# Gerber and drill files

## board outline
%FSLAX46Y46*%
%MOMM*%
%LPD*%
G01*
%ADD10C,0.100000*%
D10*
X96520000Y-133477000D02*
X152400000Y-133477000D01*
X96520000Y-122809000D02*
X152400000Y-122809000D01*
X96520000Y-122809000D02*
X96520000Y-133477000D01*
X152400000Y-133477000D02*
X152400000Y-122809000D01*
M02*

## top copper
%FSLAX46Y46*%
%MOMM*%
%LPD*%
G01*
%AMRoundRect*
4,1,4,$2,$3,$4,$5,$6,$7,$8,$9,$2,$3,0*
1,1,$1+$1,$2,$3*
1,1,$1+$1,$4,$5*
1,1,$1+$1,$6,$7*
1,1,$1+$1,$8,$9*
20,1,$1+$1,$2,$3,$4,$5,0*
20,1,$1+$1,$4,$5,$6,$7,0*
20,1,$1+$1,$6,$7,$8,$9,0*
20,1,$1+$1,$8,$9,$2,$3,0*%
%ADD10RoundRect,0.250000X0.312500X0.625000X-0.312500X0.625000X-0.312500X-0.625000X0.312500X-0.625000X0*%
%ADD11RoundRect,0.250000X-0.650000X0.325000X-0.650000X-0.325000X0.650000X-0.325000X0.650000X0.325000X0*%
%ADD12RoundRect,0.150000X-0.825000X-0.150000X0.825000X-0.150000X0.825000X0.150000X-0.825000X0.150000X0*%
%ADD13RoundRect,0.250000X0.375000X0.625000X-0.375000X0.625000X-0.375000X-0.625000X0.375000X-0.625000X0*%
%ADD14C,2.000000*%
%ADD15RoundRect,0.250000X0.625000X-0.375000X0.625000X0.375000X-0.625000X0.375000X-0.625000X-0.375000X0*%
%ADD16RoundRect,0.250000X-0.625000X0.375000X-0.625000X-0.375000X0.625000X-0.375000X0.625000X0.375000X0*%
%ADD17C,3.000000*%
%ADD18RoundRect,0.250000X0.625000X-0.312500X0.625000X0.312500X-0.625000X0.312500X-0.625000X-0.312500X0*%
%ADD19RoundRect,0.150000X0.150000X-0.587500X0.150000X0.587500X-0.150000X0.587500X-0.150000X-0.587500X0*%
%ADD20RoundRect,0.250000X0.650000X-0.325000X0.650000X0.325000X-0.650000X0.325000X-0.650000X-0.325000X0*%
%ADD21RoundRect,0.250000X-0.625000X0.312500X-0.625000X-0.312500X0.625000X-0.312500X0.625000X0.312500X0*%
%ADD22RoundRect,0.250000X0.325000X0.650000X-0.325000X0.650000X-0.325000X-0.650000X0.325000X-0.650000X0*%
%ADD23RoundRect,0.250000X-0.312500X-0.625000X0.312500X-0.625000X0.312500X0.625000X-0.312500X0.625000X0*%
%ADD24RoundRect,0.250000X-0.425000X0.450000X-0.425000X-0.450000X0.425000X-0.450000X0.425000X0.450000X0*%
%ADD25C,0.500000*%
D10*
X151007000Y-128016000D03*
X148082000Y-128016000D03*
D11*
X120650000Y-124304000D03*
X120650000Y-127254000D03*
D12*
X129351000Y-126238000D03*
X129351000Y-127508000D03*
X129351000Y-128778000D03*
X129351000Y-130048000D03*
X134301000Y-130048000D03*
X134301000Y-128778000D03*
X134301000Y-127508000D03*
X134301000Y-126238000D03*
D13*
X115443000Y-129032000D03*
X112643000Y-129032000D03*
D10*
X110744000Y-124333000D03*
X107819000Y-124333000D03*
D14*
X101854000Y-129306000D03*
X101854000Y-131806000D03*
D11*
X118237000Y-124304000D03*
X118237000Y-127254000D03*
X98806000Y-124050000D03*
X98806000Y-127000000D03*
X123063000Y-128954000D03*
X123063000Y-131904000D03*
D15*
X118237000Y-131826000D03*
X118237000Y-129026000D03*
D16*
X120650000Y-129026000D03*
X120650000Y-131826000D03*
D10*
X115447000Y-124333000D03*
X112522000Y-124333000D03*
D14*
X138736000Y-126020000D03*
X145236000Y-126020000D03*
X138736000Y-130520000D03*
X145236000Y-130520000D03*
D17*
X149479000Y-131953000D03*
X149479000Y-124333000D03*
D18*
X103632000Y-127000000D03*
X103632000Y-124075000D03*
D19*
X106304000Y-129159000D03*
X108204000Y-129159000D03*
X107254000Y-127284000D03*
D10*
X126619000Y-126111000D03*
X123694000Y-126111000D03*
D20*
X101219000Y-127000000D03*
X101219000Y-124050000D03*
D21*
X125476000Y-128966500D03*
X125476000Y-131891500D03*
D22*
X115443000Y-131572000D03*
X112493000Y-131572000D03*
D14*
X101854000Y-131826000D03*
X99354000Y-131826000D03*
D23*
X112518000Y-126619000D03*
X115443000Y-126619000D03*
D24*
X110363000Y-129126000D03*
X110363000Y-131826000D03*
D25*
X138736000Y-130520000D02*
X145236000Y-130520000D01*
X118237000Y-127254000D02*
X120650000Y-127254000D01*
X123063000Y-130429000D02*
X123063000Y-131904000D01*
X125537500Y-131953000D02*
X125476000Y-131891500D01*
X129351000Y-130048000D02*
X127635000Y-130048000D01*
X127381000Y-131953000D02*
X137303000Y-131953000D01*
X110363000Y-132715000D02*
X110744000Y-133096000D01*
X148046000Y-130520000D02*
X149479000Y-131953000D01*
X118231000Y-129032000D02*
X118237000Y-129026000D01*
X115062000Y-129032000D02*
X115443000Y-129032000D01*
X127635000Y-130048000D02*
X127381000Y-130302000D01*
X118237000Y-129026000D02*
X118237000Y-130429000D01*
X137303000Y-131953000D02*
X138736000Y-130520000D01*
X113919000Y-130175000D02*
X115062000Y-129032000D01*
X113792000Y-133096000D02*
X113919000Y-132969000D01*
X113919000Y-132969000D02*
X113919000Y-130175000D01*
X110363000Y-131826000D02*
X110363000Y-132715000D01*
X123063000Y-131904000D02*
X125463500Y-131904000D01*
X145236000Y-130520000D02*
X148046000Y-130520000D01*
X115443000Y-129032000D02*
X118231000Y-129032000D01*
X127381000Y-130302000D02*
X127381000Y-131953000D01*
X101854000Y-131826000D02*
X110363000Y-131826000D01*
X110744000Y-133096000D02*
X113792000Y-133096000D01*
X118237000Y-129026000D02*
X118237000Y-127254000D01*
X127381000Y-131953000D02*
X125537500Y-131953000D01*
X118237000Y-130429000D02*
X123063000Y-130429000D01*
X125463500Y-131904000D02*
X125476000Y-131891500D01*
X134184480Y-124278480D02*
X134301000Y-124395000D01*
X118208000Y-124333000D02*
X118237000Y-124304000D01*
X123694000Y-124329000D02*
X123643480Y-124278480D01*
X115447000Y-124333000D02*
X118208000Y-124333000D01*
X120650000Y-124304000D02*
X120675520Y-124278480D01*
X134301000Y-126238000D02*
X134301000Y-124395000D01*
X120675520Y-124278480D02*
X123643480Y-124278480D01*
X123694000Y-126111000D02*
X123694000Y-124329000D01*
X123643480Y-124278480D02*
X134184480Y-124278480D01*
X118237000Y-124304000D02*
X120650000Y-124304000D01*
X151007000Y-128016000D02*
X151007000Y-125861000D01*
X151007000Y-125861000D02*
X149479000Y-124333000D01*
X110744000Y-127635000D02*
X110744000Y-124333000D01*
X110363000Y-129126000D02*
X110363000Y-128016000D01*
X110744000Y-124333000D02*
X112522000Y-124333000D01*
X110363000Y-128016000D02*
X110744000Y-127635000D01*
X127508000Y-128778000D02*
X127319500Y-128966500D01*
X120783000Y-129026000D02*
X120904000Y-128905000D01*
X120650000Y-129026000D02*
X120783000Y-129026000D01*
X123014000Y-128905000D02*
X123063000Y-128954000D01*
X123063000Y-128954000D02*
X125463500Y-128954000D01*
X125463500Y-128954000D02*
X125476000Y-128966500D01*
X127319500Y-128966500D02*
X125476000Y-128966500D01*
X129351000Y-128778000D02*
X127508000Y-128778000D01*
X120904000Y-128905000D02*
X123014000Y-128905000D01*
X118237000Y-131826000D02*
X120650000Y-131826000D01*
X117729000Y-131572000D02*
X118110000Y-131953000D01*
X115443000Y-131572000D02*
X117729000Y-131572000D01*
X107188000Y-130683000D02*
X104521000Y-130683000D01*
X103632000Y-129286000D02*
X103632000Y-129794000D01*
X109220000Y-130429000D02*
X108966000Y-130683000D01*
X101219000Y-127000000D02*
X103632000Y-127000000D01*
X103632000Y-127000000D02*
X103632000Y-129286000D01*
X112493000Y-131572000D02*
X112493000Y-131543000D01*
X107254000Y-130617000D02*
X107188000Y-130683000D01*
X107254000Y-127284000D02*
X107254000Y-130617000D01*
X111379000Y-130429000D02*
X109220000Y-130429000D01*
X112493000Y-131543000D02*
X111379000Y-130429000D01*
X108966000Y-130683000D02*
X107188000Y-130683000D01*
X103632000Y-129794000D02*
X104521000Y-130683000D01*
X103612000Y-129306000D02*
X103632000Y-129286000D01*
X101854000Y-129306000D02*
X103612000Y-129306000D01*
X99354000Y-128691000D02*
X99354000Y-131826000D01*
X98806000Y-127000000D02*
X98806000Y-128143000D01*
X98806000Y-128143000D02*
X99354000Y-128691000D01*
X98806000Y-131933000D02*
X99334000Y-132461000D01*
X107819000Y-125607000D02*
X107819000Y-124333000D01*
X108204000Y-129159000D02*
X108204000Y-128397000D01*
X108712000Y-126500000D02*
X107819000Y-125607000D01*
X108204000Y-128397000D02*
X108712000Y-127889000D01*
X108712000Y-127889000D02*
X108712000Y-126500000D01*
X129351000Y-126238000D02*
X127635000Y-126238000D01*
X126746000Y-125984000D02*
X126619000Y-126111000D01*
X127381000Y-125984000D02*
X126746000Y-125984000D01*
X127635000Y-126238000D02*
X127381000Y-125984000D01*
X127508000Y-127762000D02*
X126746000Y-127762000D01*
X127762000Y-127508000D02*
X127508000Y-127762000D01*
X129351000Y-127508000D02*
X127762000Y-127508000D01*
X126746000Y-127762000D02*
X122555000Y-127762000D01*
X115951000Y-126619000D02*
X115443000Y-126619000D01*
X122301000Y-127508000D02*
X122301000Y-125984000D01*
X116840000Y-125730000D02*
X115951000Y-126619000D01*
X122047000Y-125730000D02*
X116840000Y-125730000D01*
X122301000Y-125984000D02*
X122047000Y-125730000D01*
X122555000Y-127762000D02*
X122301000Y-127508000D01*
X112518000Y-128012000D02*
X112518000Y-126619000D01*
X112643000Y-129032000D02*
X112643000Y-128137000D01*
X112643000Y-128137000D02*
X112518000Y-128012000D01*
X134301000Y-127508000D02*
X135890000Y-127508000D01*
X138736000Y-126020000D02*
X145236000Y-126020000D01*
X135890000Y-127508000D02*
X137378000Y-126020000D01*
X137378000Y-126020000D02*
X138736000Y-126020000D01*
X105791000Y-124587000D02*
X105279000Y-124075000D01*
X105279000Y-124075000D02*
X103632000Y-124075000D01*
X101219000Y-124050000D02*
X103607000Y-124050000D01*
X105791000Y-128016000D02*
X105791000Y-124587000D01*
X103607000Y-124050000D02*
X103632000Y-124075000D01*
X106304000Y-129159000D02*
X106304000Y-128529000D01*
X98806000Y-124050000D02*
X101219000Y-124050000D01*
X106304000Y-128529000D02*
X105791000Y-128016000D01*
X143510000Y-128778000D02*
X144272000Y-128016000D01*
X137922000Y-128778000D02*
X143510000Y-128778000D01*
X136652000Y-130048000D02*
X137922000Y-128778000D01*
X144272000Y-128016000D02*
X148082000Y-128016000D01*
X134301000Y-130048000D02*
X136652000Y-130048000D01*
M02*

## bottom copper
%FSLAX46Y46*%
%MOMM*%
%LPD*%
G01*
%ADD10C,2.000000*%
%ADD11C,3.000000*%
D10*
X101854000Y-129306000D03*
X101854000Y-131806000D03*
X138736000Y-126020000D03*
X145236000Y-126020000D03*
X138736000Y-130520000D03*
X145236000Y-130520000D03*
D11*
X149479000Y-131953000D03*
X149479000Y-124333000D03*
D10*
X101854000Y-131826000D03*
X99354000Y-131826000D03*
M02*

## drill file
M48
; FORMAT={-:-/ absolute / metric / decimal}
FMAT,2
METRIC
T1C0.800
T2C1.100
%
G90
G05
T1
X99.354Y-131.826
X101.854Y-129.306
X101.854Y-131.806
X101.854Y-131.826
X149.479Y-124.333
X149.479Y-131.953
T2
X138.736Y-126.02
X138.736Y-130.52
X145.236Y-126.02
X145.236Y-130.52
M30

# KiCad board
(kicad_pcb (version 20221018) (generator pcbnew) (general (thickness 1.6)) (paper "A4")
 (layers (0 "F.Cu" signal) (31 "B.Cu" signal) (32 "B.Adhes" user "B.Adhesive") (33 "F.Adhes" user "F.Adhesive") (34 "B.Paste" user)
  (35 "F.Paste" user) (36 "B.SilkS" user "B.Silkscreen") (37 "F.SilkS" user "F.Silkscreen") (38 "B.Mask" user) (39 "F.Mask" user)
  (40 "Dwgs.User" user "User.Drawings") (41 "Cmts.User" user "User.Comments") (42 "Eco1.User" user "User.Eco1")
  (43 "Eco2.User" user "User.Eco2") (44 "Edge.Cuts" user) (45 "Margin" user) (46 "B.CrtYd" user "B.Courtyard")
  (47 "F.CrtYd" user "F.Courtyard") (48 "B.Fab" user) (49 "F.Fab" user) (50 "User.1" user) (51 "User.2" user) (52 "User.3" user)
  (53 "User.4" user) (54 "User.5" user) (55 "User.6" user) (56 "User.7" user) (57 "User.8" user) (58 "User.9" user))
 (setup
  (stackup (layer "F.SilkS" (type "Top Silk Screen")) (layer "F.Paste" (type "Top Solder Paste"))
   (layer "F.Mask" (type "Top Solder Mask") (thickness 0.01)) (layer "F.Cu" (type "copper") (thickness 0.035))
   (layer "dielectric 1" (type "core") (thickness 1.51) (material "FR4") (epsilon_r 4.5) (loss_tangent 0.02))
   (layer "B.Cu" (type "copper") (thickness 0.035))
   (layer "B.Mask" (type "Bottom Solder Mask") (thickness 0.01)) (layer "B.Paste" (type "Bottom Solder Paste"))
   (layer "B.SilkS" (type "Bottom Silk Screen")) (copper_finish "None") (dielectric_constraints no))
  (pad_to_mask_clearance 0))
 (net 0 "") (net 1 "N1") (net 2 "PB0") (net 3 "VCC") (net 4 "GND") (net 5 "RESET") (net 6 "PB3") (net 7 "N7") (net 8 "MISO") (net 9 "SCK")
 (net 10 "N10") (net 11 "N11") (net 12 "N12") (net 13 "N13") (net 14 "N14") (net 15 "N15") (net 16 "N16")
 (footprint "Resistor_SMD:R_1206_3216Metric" (layer "F.Cu") (at 149.5445 128.016 180)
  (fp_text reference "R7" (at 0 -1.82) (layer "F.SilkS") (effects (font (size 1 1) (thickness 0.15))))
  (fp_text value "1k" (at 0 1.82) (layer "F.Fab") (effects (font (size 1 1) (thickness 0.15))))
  (pad "1" smd roundrect (at -1.4625 0 180) (size 1.125 1.75) (layers "F.Cu" "F.Paste" "F.Mask") (roundrect_rratio 0.222222) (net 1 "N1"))
  (pad "2" smd roundrect (at 1.4625 0 180) (size 1.125 1.75) (layers "F.Cu" "F.Paste" "F.Mask") (roundrect_rratio 0.222222) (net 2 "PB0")))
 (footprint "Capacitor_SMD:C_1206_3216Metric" (layer "F.Cu") (at 120.65 125.779 -90)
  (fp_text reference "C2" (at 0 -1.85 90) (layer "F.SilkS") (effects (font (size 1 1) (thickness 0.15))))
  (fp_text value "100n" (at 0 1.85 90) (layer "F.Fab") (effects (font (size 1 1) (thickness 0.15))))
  (pad "1" smd roundrect (at -1.475 0 270) (size 1.15 1.8) (layers "F.Cu" "F.Paste" "F.Mask") (roundrect_rratio 0.2173913043) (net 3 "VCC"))
  (pad "2" smd roundrect (at 1.475 0 270) (size 1.15 1.8) (layers "F.Cu" "F.Paste" "F.Mask") (roundrect_rratio 0.2173913043) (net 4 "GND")))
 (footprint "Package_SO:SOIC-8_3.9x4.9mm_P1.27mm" (layer "F.Cu") (at 131.826 128.143)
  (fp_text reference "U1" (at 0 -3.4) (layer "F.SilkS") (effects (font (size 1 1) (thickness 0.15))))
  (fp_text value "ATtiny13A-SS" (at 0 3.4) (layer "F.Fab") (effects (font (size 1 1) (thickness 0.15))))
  (pad "1" smd roundrect (at -2.475 -1.905) (size 1.95 0.6) (layers "F.Cu" "F.Paste" "F.Mask") (roundrect_rratio 0.25) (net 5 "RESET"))
  (pad "2" smd roundrect (at -2.475 -0.635) (size 1.95 0.6) (layers "F.Cu" "F.Paste" "F.Mask") (roundrect_rratio 0.25) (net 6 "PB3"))
  (pad "3" smd roundrect (at -2.475 0.635) (size 1.95 0.6) (layers "F.Cu" "F.Paste" "F.Mask") (roundrect_rratio 0.25) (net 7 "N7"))
  (pad "4" smd roundrect (at -2.475 1.905) (size 1.95 0.6) (layers "F.Cu" "F.Paste" "F.Mask") (roundrect_rratio 0.25) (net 4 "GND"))
  (pad "5" smd roundrect (at 2.475 1.905) (size 1.95 0.6) (layers "F.Cu" "F.Paste" "F.Mask") (roundrect_rratio 0.25) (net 2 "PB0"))
  (pad "6" smd roundrect (at 2.475 0.635) (size 1.95 0.6) (layers "F.Cu" "F.Paste" "F.Mask") (roundrect_rratio 0.25) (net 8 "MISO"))
  (pad "7" smd roundrect (at 2.475 -0.635) (size 1.95 0.6) (layers "F.Cu" "F.Paste" "F.Mask") (roundrect_rratio 0.25) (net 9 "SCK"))
  (pad "8" smd roundrect (at 2.475 -1.905) (size 1.95 0.6) (layers "F.Cu" "F.Paste" "F.Mask") (roundrect_rratio 0.25) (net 3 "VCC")))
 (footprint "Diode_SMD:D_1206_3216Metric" (layer "F.Cu") (at 114.043 129.032 180)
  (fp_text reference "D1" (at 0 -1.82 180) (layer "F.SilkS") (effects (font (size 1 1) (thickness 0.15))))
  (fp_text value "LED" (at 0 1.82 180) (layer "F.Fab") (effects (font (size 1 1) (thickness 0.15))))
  (pad "1" smd roundrect (at -1.4 0 180) (size 1.25 1.75) (layers "F.Cu" "F.Paste" "F.Mask") (roundrect_rratio 0.2) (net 4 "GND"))
  (pad "2" smd roundrect (at 1.4 0 180) (size 1.25 1.75) (layers "F.Cu" "F.Paste" "F.Mask") (roundrect_rratio 0.2) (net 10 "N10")))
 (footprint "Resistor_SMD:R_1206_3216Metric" (layer "F.Cu") (at 109.2815 124.333 180)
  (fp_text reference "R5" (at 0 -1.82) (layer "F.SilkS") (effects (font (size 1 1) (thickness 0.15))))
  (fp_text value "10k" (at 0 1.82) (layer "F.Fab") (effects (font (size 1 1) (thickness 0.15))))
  (pad "1" smd roundrect (at -1.4625 0 180) (size 1.125 1.75) (layers "F.Cu" "F.Paste" "F.Mask") (roundrect_rratio 0.2222222222)
   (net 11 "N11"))
  (pad "2" smd roundrect (at 1.4625 0 180) (size 1.125 1.75) (layers "F.Cu" "F.Paste" "F.Mask") (roundrect_rratio 0.2222222222)
   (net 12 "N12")))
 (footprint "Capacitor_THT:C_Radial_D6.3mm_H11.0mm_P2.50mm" (layer "F.Cu") (at 101.854 129.306 -90)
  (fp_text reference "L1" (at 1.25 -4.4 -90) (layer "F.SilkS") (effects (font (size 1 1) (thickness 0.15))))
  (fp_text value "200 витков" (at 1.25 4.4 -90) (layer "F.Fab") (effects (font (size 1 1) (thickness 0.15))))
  (pad "1" thru_hole circle (at 0 0 270) (size 2 2) (drill 0.8) (layers "*.Cu" "*.Mask") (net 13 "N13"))
  (pad "2" thru_hole circle (at 2.5 0 270) (size 2 2) (drill 0.8) (layers "*.Cu" "*.Mask") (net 4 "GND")))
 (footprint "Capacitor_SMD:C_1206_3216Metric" (layer "F.Cu") (at 118.237 125.779 -90)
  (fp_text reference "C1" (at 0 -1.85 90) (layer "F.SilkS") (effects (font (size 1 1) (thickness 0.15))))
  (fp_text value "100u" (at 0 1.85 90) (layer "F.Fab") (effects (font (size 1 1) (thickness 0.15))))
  (pad "1" smd roundrect (at -1.475 0 270) (size 1.15 1.8) (layers "F.Cu" "F.Paste" "F.Mask") (roundrect_rratio 0.2173913043) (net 3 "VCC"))
  (pad "2" smd roundrect (at 1.475 0 270) (size 1.15 1.8) (layers "F.Cu" "F.Paste" "F.Mask") (roundrect_rratio 0.2173913043) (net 4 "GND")))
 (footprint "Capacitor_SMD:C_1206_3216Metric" (layer "F.Cu") (at 98.806 125.525 -90)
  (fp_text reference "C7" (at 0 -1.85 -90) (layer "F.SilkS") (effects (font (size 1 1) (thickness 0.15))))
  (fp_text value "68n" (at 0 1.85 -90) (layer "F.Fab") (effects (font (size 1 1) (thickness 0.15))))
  (pad "1" smd roundrect (at -1.475 0 270) (size 1.15 1.8) (layers "F.Cu" "F.Paste" "F.Mask") (roundrect_rratio 0.2173913043) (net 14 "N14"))
  (pad "2" smd roundrect (at 1.475 0 270) (size 1.15 1.8) (layers "F.Cu" "F.Paste" "F.Mask") (roundrect_rratio 0.2173913043) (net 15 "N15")))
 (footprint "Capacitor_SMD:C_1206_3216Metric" (layer "F.Cu") (at 123.063 130.429 -90)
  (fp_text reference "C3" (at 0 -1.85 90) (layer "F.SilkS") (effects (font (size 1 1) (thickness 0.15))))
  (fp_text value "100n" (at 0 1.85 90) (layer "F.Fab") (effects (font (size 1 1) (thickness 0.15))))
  (pad "1" smd roundrect (at -1.475 0 270) (size 1.15 1.8) (layers "F.Cu" "F.Paste" "F.Mask") (roundrect_rratio 0.2173913043) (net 7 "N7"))
  (pad "2" smd roundrect (at 1.475 0 270) (size 1.15 1.8) (layers "F.Cu" "F.Paste" "F.Mask") (roundrect_rratio 0.2173913043) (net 4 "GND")))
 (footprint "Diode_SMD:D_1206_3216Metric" (layer "F.Cu") (at 118.237 130.426 90)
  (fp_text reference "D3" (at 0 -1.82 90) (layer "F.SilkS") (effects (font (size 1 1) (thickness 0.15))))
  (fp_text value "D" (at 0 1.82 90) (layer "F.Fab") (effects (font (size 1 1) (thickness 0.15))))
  (pad "1" smd roundrect (at -1.4 0 90) (size 1.25 1.75) (layers "F.Cu" "F.Paste" "F.Mask") (roundrect_rratio 0.2) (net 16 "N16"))
  (pad "2" smd roundrect (at 1.4 0 90) (size 1.25 1.75) (layers "F.Cu" "F.Paste" "F.Mask") (roundrect_rratio 0.2) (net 4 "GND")))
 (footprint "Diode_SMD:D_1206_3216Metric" (layer "F.Cu") (at 120.65 130.426 -90)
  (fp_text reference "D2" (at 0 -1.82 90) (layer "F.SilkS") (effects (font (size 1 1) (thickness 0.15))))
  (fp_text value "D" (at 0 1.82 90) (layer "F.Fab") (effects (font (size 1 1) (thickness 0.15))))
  (pad "1" smd roundrect (at -1.4 0 270) (size 1.25 1.75) (layers "F.Cu" "F.Paste" "F.Mask") (roundrect_rratio 0.2) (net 7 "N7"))
  (pad "2" smd roundrect (at 1.4 0 270) (size 1.25 1.75) (layers "F.Cu" "F.Paste" "F.Mask") (roundrect_rratio 0.2) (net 16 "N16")))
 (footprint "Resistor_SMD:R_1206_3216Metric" (layer "F.Cu") (at 113.9845 124.333 180)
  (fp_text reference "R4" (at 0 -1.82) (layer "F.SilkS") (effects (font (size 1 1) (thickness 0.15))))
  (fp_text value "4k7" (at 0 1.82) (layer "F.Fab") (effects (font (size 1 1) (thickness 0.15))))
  (pad "1" smd roundrect (at -1.4625 0 180) (size 1.125 1.75) (layers "F.Cu" "F.Paste" "F.Mask") (roundrect_rratio 0.2222222222)
   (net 3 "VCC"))
  (pad "2" smd roundrect (at 1.4625 0 180) (size 1.125 1.75) (layers "F.Cu" "F.Paste" "F.Mask") (roundrect_rratio 0.2222222222)
   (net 11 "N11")))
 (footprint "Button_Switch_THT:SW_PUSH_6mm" (layer "F.Cu") (at 138.736 126.02)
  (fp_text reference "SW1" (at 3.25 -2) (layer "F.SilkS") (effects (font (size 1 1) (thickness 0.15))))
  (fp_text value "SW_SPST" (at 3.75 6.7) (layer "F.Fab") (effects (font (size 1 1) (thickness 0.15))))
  (pad "1" thru_hole circle (at 0 0 90) (size 2 2) (drill 1.1) (layers "*.Cu" "*.Mask") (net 9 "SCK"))
  (pad "1" thru_hole circle (at 6.5 0 90) (size 2 2) (drill 1.1) (layers "*.Cu" "*.Mask") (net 9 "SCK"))
  (pad "2" thru_hole circle (at 0 4.5 90) (size 2 2) (drill 1.1) (layers "*.Cu" "*.Mask") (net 4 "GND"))
  (pad "2" thru_hole circle (at 6.5 4.5 90) (size 2 2) (drill 1.1) (layers "*.Cu" "*.Mask") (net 4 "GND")))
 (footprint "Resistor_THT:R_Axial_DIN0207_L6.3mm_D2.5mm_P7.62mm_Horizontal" (layer "F.Cu") (at 149.479 131.953 90)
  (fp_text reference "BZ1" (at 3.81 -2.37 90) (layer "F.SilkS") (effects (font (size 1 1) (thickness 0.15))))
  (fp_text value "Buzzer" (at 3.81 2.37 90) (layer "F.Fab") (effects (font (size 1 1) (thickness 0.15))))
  (pad "1" thru_hole circle (at 0 0 90) (size 3 3) (drill 0.8) (layers "*.Cu" "*.Mask") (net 4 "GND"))
  (pad "2" thru_hole circle (at 7.62 0 90) (size 3 3) (drill 0.8) (layers "*.Cu" "*.Mask") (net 1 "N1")))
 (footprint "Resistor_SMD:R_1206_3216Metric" (layer "F.Cu") (at 103.632 125.5375 90)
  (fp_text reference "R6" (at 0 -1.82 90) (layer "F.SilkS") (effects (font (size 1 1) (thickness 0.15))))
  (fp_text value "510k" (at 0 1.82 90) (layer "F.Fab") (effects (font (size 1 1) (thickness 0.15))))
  (pad "1" smd roundrect (at -1.4625 0 90) (size 1.125 1.75) (layers "F.Cu" "F.Paste" "F.Mask") (roundrect_rratio 0.2222222222)
   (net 13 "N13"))
  (pad "2" smd roundrect (at 1.4625 0 90) (size 1.125 1.75) (layers "F.Cu" "F.Paste" "F.Mask") (roundrect_rratio 0.2222222222)
   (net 14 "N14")))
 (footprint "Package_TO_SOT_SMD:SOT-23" (layer "F.Cu") (at 107.254 128.2215 90)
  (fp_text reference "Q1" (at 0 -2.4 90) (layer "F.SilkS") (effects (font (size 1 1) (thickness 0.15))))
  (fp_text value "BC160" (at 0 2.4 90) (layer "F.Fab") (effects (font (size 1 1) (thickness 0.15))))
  (pad "1" smd roundrect (at -0.9375 -0.95 90) (size 1.475 0.6) (layers "F.Cu" "F.Paste" "F.Mask") (roundrect_rratio 0.25) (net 14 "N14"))
  (pad "2" smd roundrect (at -0.9375 0.95 90) (size 1.475 0.6) (layers "F.Cu" "F.Paste" "F.Mask") (roundrect_rratio 0.25) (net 12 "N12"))
  (pad "3" smd roundrect (at 0.9375 0 90) (size 1.475 0.6) (layers "F.Cu" "F.Paste" "F.Mask") (roundrect_rratio 0.25) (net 13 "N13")))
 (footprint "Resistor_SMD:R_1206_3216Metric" (layer "F.Cu") (at 125.1565 126.111 180)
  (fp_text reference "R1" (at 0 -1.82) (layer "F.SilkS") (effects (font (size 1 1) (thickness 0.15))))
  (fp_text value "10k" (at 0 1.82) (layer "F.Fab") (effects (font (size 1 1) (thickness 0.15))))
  (pad "1" smd roundrect (at -1.4625 0 180) (size 1.125 1.75) (layers "F.Cu" "F.Paste" "F.Mask") (roundrect_rratio 0.2222222222)
   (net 5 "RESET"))
  (pad "2" smd roundrect (at 1.4625 0 180) (size 1.125 1.75) (layers "F.Cu" "F.Paste" "F.Mask") (roundrect_rratio 0.2222222222)
   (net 3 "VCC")))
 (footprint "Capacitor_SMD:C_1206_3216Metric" (layer "F.Cu") (at 101.219 125.525 90)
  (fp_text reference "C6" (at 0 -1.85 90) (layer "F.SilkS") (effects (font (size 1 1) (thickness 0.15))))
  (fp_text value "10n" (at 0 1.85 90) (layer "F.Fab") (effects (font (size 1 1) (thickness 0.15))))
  (pad "1" smd roundrect (at -1.475 0 90) (size 1.15 1.8) (layers "F.Cu" "F.Paste" "F.Mask") (roundrect_rratio 0.2173913043) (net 13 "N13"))
  (pad "2" smd roundrect (at 1.475 0 90) (size 1.15 1.8) (layers "F.Cu" "F.Paste" "F.Mask") (roundrect_rratio 0.2173913043) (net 14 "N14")))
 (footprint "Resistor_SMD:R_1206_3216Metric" (layer "F.Cu") (at 125.476 130.429 -90)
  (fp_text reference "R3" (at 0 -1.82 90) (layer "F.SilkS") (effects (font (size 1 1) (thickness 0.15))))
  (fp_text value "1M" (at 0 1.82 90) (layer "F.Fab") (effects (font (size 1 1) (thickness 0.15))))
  (pad "1" smd roundrect (at -1.4625 0 270) (size 1.125 1.75) (layers "F.Cu" "F.Paste" "F.Mask") (roundrect_rratio 0.2222222222)
   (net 7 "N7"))
  (pad "2" smd roundrect (at 1.4625 0 270) (size 1.125 1.75) (layers "F.Cu" "F.Paste" "F.Mask") (roundrect_rratio 0.2222222222)
   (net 4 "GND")))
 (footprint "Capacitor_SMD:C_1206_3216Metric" (layer "F.Cu") (at 113.968 131.572 180)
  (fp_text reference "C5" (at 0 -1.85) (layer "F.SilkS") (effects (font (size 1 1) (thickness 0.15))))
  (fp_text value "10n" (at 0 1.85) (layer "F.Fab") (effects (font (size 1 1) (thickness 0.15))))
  (pad "1" smd roundrect (at -1.475 0 180) (size 1.15 1.8) (layers "F.Cu" "F.Paste" "F.Mask") (roundrect_rratio 0.2173913043) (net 16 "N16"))
  (pad "2" smd roundrect (at 1.475 0 180) (size 1.15 1.8) (layers "F.Cu" "F.Paste" "F.Mask") (roundrect_rratio 0.2173913043) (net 13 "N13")))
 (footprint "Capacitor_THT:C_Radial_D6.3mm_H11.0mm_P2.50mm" (layer "F.Cu") (at 101.854 131.826 180)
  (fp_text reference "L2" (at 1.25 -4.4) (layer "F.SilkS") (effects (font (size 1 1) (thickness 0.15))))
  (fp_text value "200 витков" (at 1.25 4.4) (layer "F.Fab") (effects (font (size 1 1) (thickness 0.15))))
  (pad "1" thru_hole circle (at 0 0 180) (size 2 2) (drill 0.8) (layers "*.Cu" "*.Mask") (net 4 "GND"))
  (pad "2" thru_hole circle (at 2.5 0 180) (size 2 2) (drill 0.8) (layers "*.Cu" "*.Mask") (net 15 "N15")))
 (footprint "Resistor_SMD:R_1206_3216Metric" (layer "F.Cu") (at 113.9805 126.619)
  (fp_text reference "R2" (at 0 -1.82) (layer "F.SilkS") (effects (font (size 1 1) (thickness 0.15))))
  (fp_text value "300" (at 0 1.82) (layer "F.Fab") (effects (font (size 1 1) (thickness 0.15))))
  (pad "1" smd roundrect (at -1.4625 0) (size 1.125 1.75) (layers "F.Cu" "F.Paste" "F.Mask") (roundrect_rratio 0.2222222222) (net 10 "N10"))
  (pad "2" smd roundrect (at 1.4625 0) (size 1.125 1.75) (layers "F.Cu" "F.Paste" "F.Mask") (roundrect_rratio 0.2222222222) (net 6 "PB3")))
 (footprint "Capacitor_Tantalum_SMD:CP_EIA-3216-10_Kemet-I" (layer "F.Cu") (at 110.363 130.476 -90)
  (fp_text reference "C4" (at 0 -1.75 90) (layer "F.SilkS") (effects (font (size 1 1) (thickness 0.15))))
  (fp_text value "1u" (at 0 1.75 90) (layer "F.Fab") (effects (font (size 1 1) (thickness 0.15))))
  (pad "1" smd roundrect (at -1.35 0 270) (size 1.4 1.35) (layers "F.Cu" "F.Paste" "F.Mask") (roundrect_rratio 0.1851851852) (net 11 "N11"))
  (pad "2" smd roundrect (at 1.35 0 270) (size 1.4 1.35) (layers "F.Cu" "F.Paste" "F.Mask") (roundrect_rratio 0.1851851852) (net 4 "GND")))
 (gr_line (start 96.52 133.477) (end 152.4 133.477) (stroke (width 0.1) (type solid)) (layer "Edge.Cuts"))
 (gr_line (start 96.52 122.809) (end 152.4 122.809) (stroke (width 0.1) (type solid)) (layer "Edge.Cuts"))
 (gr_line (start 96.52 122.809) (end 96.52 133.477) (stroke (width 0.1) (type solid)) (layer "Edge.Cuts"))
 (gr_line (start 152.4 133.477) (end 152.4 122.809) (stroke (width 0.1) (type solid)) (layer "Edge.Cuts"))
 (segment (start 138.736 130.52) (end 145.236 130.52) (width 0.5) (layer "F.Cu") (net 4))
 (segment (start 118.237 127.254) (end 120.65 127.254) (width 0.5) (layer "F.Cu") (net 4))
 (segment (start 123.063 130.429) (end 123.063 131.904) (width 0.5) (layer "F.Cu") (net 4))
 (segment (start 125.5375 131.953) (end 125.476 131.8915) (width 0.5) (layer "F.Cu") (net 4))
 (segment (start 129.351 130.048) (end 127.635 130.048) (width 0.5) (layer "F.Cu") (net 4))
 (segment (start 127.381 131.953) (end 137.303 131.953) (width 0.5) (layer "F.Cu") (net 4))
 (segment (start 110.363 132.715) (end 110.744 133.096) (width 0.5) (layer "F.Cu") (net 4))
 (segment (start 148.046 130.52) (end 149.479 131.953) (width 0.5) (layer "F.Cu") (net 4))
 (segment (start 118.231 129.032) (end 118.237 129.026) (width 0.5) (layer "F.Cu") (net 4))
 (segment (start 115.062 129.032) (end 115.443 129.032) (width 0.5) (layer "F.Cu") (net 4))
 (segment (start 127.635 130.048) (end 127.381 130.302) (width 0.5) (layer "F.Cu") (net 4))
 (segment (start 118.237 129.026) (end 118.237 130.429) (width 0.5) (layer "F.Cu") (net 4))
 (segment (start 137.303 131.953) (end 138.736 130.52) (width 0.5) (layer "F.Cu") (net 4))
 (segment (start 113.919 130.175) (end 115.062 129.032) (width 0.5) (layer "F.Cu") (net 4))
 (segment (start 113.792 133.096) (end 113.919 132.969) (width 0.5) (layer "F.Cu") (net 4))
 (segment (start 113.919 132.969) (end 113.919 130.175) (width 0.5) (layer "F.Cu") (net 4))
 (segment (start 110.363 131.826) (end 110.363 132.715) (width 0.5) (layer "F.Cu") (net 4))
 (segment (start 123.063 131.904) (end 125.4635 131.904) (width 0.5) (layer "F.Cu") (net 4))
 (segment (start 145.236 130.52) (end 148.046 130.52) (width 0.5) (layer "F.Cu") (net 4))
 (segment (start 115.443 129.032) (end 118.231 129.032) (width 0.5) (layer "F.Cu") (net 4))
 (segment (start 127.381 130.302) (end 127.381 131.953) (width 0.5) (layer "F.Cu") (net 4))
 (segment (start 101.854 131.826) (end 110.363 131.826) (width 0.5) (layer "F.Cu") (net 4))
 (segment (start 110.744 133.096) (end 113.792 133.096) (width 0.5) (layer "F.Cu") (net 4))
 (segment (start 118.237 129.026) (end 118.237 127.254) (width 0.5) (layer "F.Cu") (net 4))
 (segment (start 127.381 131.953) (end 125.5375 131.953) (width 0.5) (layer "F.Cu") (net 4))
 (segment (start 118.237 130.429) (end 123.063 130.429) (width 0.5) (layer "F.Cu") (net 4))
 (segment (start 125.4635 131.904) (end 125.476 131.8915) (width 0.5) (layer "F.Cu") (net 4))
 (segment (start 134.18448 124.27848) (end 134.301 124.395) (width 0.5) (layer "F.Cu") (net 3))
 (segment (start 118.208 124.333) (end 118.237 124.304) (width 0.5) (layer "F.Cu") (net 3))
 (segment (start 123.694 124.329) (end 123.64348 124.27848) (width 0.5) (layer "F.Cu") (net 3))
 (segment (start 115.447 124.333) (end 118.208 124.333) (width 0.5) (layer "F.Cu") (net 3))
 (segment (start 120.65 124.304) (end 120.67552 124.27848) (width 0.5) (layer "F.Cu") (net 3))
 (segment (start 134.301 126.238) (end 134.301 124.395) (width 0.5) (layer "F.Cu") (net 3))
 (segment (start 120.67552 124.27848) (end 123.64348 124.27848) (width 0.5) (layer "F.Cu") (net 3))
 (segment (start 123.694 126.111) (end 123.694 124.329) (width 0.5) (layer "F.Cu") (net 3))
 (segment (start 123.64348 124.27848) (end 134.18448 124.27848) (width 0.5) (layer "F.Cu") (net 3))
 (segment (start 118.237 124.304) (end 120.65 124.304) (width 0.5) (layer "F.Cu") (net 3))
 (segment (start 151.007 128.016) (end 151.007 125.861) (width 0.5) (layer "F.Cu") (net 1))
 (segment (start 151.007 125.861) (end 149.479 124.333) (width 0.5) (layer "F.Cu") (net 1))
 (segment (start 110.744 127.635) (end 110.744 124.333) (width 0.5) (layer "F.Cu") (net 11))
 (segment (start 110.363 129.126) (end 110.363 128.016) (width 0.5) (layer "F.Cu") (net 11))
 (segment (start 110.744 124.333) (end 112.522 124.333) (width 0.5) (layer "F.Cu") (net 11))
 (segment (start 110.363 128.016) (end 110.744 127.635) (width 0.5) (layer "F.Cu") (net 11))
 (segment (start 127.508 128.778) (end 127.3195 128.9665) (width 0.5) (layer "F.Cu") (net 7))
 (segment (start 120.783 129.026) (end 120.904 128.905) (width 0.5) (layer "F.Cu") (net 7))
 (segment (start 120.65 129.026) (end 120.783 129.026) (width 0.5) (layer "F.Cu") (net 7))
 (segment (start 123.014 128.905) (end 123.063 128.954) (width 0.5) (layer "F.Cu") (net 7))
 (segment (start 123.063 128.954) (end 125.4635 128.954) (width 0.5) (layer "F.Cu") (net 7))
 (segment (start 125.4635 128.954) (end 125.476 128.9665) (width 0.5) (layer "F.Cu") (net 7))
 (segment (start 127.3195 128.9665) (end 125.476 128.9665) (width 0.5) (layer "F.Cu") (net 7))
 (segment (start 129.351 128.778) (end 127.508 128.778) (width 0.5) (layer "F.Cu") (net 7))
 (segment (start 120.904 128.905) (end 123.014 128.905) (width 0.5) (layer "F.Cu") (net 7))
 (segment (start 118.237 131.826) (end 120.65 131.826) (width 0.5) (layer "F.Cu") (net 16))
 (segment (start 117.729 131.572) (end 118.11 131.953) (width 0.5) (layer "F.Cu") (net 16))
 (segment (start 115.443 131.572) (end 117.729 131.572) (width 0.5) (layer "F.Cu") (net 16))
 (segment (start 107.188 130.683) (end 104.521 130.683) (width 0.5) (layer "F.Cu") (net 13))
 (segment (start 103.632 129.286) (end 103.632 129.794) (width 0.5) (layer "F.Cu") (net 13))
 (segment (start 109.22 130.429) (end 108.966 130.683) (width 0.5) (layer "F.Cu") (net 13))
 (segment (start 101.219 127) (end 103.632 127) (width 0.5) (layer "F.Cu") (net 13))
 (segment (start 103.632 127) (end 103.632 129.286) (width 0.5) (layer "F.Cu") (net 13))
 (segment (start 112.493 131.572) (end 112.493 131.543) (width 0.5) (layer "F.Cu") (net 13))
 (segment (start 107.254 130.617) (end 107.188 130.683) (width 0.5) (layer "F.Cu") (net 13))
 (segment (start 107.254 127.284) (end 107.254 130.617) (width 0.5) (layer "F.Cu") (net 13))
 (segment (start 111.379 130.429) (end 109.22 130.429) (width 0.5) (layer "F.Cu") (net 13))
 (segment (start 112.493 131.543) (end 111.379 130.429) (width 0.5) (layer "F.Cu") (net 13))
 (segment (start 108.966 130.683) (end 107.188 130.683) (width 0.5) (layer "F.Cu") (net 13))
 (segment (start 103.632 129.794) (end 104.521 130.683) (width 0.5) (layer "F.Cu") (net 13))
 (segment (start 103.612 129.306) (end 103.632 129.286) (width 0.5) (layer "F.Cu") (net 13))
 (segment (start 101.854 129.306) (end 103.612 129.306) (width 0.5) (layer "F.Cu") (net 13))
 (segment (start 99.354 128.691) (end 99.354 131.826) (width 0.5) (layer "F.Cu") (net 15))
 (segment (start 98.806 127) (end 98.806 128.143) (width 0.5) (layer "F.Cu") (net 15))
 (segment (start 98.806 128.143) (end 99.354 128.691) (width 0.5) (layer "F.Cu") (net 15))
 (segment (start 98.806 131.933) (end 99.334 132.461) (width 0.5) (layer "F.Cu") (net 15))
 (segment (start 107.819 125.607) (end 107.819 124.333) (width 0.5) (layer "F.Cu") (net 12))
 (segment (start 108.204 129.159) (end 108.204 128.397) (width 0.5) (layer "F.Cu") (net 12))
 (segment (start 108.712 126.5) (end 107.819 125.607) (width 0.5) (layer "F.Cu") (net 12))
 (segment (start 108.204 128.397) (end 108.712 127.889) (width 0.5) (layer "F.Cu") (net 12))
 (segment (start 108.712 127.889) (end 108.712 126.5) (width 0.5) (layer "F.Cu") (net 12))
 (segment (start 129.351 126.238) (end 127.635 126.238) (width 0.5) (layer "F.Cu") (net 5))
 (segment (start 126.746 125.984) (end 126.619 126.111) (width 0.5) (layer "F.Cu") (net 5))
 (segment (start 127.381 125.984) (end 126.746 125.984) (width 0.5) (layer "F.Cu") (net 5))
 (segment (start 127.635 126.238) (end 127.381 125.984) (width 0.5) (layer "F.Cu") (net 5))
 (segment (start 127.508 127.762) (end 126.746 127.762) (width 0.5) (layer "F.Cu") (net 6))
 (segment (start 127.762 127.508) (end 127.508 127.762) (width 0.5) (layer "F.Cu") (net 6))
 (segment (start 129.351 127.508) (end 127.762 127.508) (width 0.5) (layer "F.Cu") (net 6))
 (segment (start 126.746 127.762) (end 122.555 127.762) (width 0.5) (layer "F.Cu") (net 6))
 (segment (start 115.951 126.619) (end 115.443 126.619) (width 0.5) (layer "F.Cu") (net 6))
 (segment (start 122.301 127.508) (end 122.301 125.984) (width 0.5) (layer "F.Cu") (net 6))
 (segment (start 116.84 125.73) (end 115.951 126.619) (width 0.5) (layer "F.Cu") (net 6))
 (segment (start 122.047 125.73) (end 116.84 125.73) (width 0.5) (layer "F.Cu") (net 6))
 (segment (start 122.301 125.984) (end 122.047 125.73) (width 0.5) (layer "F.Cu") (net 6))
 (segment (start 122.555 127.762) (end 122.301 127.508) (width 0.5) (layer "F.Cu") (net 6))
 (segment (start 112.518 128.012) (end 112.518 126.619) (width 0.5) (layer "F.Cu") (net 10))
 (segment (start 112.643 129.032) (end 112.643 128.137) (width 0.5) (layer "F.Cu") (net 10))
 (segment (start 112.643 128.137) (end 112.518 128.012) (width 0.5) (layer "F.Cu") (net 10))
 (segment (start 134.301 127.508) (end 135.89 127.508) (width 0.5) (layer "F.Cu") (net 9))
 (segment (start 138.736 126.02) (end 145.236 126.02) (width 0.5) (layer "F.Cu") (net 9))
 (segment (start 135.89 127.508) (end 137.378 126.02) (width 0.5) (layer "F.Cu") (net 9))
 (segment (start 137.378 126.02) (end 138.736 126.02) (width 0.5) (layer "F.Cu") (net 9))
 (segment (start 105.791 124.587) (end 105.279 124.075) (width 0.5) (layer "F.Cu") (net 14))
 (segment (start 105.279 124.075) (end 103.632 124.075) (width 0.5) (layer "F.Cu") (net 14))
 (segment (start 101.219 124.05) (end 103.607 124.05) (width 0.5) (layer "F.Cu") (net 14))
 (segment (start 105.791 128.016) (end 105.791 124.587) (width 0.5) (layer "F.Cu") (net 14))
 (segment (start 103.607 124.05) (end 103.632 124.075) (width 0.5) (layer "F.Cu") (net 14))
 (segment (start 106.304 129.159) (end 106.304 128.529) (width 0.5) (layer "F.Cu") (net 14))
 (segment (start 98.806 124.05) (end 101.219 124.05) (width 0.5) (layer "F.Cu") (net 14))
 (segment (start 106.304 128.529) (end 105.791 128.016) (width 0.5) (layer "F.Cu") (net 14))
 (segment (start 143.51 128.778) (end 144.272 128.016) (width 0.5) (layer "F.Cu") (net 2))
 (segment (start 137.922 128.778) (end 143.51 128.778) (width 0.5) (layer "F.Cu") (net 2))
 (segment (start 136.652 130.048) (end 137.922 128.778) (width 0.5) (layer "F.Cu") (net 2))
 (segment (start 144.272 128.016) (end 148.082 128.016) (width 0.5) (layer "F.Cu") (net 2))
 (segment (start 134.301 130.048) (end 136.652 130.048) (width 0.5) (layer "F.Cu") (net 2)))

